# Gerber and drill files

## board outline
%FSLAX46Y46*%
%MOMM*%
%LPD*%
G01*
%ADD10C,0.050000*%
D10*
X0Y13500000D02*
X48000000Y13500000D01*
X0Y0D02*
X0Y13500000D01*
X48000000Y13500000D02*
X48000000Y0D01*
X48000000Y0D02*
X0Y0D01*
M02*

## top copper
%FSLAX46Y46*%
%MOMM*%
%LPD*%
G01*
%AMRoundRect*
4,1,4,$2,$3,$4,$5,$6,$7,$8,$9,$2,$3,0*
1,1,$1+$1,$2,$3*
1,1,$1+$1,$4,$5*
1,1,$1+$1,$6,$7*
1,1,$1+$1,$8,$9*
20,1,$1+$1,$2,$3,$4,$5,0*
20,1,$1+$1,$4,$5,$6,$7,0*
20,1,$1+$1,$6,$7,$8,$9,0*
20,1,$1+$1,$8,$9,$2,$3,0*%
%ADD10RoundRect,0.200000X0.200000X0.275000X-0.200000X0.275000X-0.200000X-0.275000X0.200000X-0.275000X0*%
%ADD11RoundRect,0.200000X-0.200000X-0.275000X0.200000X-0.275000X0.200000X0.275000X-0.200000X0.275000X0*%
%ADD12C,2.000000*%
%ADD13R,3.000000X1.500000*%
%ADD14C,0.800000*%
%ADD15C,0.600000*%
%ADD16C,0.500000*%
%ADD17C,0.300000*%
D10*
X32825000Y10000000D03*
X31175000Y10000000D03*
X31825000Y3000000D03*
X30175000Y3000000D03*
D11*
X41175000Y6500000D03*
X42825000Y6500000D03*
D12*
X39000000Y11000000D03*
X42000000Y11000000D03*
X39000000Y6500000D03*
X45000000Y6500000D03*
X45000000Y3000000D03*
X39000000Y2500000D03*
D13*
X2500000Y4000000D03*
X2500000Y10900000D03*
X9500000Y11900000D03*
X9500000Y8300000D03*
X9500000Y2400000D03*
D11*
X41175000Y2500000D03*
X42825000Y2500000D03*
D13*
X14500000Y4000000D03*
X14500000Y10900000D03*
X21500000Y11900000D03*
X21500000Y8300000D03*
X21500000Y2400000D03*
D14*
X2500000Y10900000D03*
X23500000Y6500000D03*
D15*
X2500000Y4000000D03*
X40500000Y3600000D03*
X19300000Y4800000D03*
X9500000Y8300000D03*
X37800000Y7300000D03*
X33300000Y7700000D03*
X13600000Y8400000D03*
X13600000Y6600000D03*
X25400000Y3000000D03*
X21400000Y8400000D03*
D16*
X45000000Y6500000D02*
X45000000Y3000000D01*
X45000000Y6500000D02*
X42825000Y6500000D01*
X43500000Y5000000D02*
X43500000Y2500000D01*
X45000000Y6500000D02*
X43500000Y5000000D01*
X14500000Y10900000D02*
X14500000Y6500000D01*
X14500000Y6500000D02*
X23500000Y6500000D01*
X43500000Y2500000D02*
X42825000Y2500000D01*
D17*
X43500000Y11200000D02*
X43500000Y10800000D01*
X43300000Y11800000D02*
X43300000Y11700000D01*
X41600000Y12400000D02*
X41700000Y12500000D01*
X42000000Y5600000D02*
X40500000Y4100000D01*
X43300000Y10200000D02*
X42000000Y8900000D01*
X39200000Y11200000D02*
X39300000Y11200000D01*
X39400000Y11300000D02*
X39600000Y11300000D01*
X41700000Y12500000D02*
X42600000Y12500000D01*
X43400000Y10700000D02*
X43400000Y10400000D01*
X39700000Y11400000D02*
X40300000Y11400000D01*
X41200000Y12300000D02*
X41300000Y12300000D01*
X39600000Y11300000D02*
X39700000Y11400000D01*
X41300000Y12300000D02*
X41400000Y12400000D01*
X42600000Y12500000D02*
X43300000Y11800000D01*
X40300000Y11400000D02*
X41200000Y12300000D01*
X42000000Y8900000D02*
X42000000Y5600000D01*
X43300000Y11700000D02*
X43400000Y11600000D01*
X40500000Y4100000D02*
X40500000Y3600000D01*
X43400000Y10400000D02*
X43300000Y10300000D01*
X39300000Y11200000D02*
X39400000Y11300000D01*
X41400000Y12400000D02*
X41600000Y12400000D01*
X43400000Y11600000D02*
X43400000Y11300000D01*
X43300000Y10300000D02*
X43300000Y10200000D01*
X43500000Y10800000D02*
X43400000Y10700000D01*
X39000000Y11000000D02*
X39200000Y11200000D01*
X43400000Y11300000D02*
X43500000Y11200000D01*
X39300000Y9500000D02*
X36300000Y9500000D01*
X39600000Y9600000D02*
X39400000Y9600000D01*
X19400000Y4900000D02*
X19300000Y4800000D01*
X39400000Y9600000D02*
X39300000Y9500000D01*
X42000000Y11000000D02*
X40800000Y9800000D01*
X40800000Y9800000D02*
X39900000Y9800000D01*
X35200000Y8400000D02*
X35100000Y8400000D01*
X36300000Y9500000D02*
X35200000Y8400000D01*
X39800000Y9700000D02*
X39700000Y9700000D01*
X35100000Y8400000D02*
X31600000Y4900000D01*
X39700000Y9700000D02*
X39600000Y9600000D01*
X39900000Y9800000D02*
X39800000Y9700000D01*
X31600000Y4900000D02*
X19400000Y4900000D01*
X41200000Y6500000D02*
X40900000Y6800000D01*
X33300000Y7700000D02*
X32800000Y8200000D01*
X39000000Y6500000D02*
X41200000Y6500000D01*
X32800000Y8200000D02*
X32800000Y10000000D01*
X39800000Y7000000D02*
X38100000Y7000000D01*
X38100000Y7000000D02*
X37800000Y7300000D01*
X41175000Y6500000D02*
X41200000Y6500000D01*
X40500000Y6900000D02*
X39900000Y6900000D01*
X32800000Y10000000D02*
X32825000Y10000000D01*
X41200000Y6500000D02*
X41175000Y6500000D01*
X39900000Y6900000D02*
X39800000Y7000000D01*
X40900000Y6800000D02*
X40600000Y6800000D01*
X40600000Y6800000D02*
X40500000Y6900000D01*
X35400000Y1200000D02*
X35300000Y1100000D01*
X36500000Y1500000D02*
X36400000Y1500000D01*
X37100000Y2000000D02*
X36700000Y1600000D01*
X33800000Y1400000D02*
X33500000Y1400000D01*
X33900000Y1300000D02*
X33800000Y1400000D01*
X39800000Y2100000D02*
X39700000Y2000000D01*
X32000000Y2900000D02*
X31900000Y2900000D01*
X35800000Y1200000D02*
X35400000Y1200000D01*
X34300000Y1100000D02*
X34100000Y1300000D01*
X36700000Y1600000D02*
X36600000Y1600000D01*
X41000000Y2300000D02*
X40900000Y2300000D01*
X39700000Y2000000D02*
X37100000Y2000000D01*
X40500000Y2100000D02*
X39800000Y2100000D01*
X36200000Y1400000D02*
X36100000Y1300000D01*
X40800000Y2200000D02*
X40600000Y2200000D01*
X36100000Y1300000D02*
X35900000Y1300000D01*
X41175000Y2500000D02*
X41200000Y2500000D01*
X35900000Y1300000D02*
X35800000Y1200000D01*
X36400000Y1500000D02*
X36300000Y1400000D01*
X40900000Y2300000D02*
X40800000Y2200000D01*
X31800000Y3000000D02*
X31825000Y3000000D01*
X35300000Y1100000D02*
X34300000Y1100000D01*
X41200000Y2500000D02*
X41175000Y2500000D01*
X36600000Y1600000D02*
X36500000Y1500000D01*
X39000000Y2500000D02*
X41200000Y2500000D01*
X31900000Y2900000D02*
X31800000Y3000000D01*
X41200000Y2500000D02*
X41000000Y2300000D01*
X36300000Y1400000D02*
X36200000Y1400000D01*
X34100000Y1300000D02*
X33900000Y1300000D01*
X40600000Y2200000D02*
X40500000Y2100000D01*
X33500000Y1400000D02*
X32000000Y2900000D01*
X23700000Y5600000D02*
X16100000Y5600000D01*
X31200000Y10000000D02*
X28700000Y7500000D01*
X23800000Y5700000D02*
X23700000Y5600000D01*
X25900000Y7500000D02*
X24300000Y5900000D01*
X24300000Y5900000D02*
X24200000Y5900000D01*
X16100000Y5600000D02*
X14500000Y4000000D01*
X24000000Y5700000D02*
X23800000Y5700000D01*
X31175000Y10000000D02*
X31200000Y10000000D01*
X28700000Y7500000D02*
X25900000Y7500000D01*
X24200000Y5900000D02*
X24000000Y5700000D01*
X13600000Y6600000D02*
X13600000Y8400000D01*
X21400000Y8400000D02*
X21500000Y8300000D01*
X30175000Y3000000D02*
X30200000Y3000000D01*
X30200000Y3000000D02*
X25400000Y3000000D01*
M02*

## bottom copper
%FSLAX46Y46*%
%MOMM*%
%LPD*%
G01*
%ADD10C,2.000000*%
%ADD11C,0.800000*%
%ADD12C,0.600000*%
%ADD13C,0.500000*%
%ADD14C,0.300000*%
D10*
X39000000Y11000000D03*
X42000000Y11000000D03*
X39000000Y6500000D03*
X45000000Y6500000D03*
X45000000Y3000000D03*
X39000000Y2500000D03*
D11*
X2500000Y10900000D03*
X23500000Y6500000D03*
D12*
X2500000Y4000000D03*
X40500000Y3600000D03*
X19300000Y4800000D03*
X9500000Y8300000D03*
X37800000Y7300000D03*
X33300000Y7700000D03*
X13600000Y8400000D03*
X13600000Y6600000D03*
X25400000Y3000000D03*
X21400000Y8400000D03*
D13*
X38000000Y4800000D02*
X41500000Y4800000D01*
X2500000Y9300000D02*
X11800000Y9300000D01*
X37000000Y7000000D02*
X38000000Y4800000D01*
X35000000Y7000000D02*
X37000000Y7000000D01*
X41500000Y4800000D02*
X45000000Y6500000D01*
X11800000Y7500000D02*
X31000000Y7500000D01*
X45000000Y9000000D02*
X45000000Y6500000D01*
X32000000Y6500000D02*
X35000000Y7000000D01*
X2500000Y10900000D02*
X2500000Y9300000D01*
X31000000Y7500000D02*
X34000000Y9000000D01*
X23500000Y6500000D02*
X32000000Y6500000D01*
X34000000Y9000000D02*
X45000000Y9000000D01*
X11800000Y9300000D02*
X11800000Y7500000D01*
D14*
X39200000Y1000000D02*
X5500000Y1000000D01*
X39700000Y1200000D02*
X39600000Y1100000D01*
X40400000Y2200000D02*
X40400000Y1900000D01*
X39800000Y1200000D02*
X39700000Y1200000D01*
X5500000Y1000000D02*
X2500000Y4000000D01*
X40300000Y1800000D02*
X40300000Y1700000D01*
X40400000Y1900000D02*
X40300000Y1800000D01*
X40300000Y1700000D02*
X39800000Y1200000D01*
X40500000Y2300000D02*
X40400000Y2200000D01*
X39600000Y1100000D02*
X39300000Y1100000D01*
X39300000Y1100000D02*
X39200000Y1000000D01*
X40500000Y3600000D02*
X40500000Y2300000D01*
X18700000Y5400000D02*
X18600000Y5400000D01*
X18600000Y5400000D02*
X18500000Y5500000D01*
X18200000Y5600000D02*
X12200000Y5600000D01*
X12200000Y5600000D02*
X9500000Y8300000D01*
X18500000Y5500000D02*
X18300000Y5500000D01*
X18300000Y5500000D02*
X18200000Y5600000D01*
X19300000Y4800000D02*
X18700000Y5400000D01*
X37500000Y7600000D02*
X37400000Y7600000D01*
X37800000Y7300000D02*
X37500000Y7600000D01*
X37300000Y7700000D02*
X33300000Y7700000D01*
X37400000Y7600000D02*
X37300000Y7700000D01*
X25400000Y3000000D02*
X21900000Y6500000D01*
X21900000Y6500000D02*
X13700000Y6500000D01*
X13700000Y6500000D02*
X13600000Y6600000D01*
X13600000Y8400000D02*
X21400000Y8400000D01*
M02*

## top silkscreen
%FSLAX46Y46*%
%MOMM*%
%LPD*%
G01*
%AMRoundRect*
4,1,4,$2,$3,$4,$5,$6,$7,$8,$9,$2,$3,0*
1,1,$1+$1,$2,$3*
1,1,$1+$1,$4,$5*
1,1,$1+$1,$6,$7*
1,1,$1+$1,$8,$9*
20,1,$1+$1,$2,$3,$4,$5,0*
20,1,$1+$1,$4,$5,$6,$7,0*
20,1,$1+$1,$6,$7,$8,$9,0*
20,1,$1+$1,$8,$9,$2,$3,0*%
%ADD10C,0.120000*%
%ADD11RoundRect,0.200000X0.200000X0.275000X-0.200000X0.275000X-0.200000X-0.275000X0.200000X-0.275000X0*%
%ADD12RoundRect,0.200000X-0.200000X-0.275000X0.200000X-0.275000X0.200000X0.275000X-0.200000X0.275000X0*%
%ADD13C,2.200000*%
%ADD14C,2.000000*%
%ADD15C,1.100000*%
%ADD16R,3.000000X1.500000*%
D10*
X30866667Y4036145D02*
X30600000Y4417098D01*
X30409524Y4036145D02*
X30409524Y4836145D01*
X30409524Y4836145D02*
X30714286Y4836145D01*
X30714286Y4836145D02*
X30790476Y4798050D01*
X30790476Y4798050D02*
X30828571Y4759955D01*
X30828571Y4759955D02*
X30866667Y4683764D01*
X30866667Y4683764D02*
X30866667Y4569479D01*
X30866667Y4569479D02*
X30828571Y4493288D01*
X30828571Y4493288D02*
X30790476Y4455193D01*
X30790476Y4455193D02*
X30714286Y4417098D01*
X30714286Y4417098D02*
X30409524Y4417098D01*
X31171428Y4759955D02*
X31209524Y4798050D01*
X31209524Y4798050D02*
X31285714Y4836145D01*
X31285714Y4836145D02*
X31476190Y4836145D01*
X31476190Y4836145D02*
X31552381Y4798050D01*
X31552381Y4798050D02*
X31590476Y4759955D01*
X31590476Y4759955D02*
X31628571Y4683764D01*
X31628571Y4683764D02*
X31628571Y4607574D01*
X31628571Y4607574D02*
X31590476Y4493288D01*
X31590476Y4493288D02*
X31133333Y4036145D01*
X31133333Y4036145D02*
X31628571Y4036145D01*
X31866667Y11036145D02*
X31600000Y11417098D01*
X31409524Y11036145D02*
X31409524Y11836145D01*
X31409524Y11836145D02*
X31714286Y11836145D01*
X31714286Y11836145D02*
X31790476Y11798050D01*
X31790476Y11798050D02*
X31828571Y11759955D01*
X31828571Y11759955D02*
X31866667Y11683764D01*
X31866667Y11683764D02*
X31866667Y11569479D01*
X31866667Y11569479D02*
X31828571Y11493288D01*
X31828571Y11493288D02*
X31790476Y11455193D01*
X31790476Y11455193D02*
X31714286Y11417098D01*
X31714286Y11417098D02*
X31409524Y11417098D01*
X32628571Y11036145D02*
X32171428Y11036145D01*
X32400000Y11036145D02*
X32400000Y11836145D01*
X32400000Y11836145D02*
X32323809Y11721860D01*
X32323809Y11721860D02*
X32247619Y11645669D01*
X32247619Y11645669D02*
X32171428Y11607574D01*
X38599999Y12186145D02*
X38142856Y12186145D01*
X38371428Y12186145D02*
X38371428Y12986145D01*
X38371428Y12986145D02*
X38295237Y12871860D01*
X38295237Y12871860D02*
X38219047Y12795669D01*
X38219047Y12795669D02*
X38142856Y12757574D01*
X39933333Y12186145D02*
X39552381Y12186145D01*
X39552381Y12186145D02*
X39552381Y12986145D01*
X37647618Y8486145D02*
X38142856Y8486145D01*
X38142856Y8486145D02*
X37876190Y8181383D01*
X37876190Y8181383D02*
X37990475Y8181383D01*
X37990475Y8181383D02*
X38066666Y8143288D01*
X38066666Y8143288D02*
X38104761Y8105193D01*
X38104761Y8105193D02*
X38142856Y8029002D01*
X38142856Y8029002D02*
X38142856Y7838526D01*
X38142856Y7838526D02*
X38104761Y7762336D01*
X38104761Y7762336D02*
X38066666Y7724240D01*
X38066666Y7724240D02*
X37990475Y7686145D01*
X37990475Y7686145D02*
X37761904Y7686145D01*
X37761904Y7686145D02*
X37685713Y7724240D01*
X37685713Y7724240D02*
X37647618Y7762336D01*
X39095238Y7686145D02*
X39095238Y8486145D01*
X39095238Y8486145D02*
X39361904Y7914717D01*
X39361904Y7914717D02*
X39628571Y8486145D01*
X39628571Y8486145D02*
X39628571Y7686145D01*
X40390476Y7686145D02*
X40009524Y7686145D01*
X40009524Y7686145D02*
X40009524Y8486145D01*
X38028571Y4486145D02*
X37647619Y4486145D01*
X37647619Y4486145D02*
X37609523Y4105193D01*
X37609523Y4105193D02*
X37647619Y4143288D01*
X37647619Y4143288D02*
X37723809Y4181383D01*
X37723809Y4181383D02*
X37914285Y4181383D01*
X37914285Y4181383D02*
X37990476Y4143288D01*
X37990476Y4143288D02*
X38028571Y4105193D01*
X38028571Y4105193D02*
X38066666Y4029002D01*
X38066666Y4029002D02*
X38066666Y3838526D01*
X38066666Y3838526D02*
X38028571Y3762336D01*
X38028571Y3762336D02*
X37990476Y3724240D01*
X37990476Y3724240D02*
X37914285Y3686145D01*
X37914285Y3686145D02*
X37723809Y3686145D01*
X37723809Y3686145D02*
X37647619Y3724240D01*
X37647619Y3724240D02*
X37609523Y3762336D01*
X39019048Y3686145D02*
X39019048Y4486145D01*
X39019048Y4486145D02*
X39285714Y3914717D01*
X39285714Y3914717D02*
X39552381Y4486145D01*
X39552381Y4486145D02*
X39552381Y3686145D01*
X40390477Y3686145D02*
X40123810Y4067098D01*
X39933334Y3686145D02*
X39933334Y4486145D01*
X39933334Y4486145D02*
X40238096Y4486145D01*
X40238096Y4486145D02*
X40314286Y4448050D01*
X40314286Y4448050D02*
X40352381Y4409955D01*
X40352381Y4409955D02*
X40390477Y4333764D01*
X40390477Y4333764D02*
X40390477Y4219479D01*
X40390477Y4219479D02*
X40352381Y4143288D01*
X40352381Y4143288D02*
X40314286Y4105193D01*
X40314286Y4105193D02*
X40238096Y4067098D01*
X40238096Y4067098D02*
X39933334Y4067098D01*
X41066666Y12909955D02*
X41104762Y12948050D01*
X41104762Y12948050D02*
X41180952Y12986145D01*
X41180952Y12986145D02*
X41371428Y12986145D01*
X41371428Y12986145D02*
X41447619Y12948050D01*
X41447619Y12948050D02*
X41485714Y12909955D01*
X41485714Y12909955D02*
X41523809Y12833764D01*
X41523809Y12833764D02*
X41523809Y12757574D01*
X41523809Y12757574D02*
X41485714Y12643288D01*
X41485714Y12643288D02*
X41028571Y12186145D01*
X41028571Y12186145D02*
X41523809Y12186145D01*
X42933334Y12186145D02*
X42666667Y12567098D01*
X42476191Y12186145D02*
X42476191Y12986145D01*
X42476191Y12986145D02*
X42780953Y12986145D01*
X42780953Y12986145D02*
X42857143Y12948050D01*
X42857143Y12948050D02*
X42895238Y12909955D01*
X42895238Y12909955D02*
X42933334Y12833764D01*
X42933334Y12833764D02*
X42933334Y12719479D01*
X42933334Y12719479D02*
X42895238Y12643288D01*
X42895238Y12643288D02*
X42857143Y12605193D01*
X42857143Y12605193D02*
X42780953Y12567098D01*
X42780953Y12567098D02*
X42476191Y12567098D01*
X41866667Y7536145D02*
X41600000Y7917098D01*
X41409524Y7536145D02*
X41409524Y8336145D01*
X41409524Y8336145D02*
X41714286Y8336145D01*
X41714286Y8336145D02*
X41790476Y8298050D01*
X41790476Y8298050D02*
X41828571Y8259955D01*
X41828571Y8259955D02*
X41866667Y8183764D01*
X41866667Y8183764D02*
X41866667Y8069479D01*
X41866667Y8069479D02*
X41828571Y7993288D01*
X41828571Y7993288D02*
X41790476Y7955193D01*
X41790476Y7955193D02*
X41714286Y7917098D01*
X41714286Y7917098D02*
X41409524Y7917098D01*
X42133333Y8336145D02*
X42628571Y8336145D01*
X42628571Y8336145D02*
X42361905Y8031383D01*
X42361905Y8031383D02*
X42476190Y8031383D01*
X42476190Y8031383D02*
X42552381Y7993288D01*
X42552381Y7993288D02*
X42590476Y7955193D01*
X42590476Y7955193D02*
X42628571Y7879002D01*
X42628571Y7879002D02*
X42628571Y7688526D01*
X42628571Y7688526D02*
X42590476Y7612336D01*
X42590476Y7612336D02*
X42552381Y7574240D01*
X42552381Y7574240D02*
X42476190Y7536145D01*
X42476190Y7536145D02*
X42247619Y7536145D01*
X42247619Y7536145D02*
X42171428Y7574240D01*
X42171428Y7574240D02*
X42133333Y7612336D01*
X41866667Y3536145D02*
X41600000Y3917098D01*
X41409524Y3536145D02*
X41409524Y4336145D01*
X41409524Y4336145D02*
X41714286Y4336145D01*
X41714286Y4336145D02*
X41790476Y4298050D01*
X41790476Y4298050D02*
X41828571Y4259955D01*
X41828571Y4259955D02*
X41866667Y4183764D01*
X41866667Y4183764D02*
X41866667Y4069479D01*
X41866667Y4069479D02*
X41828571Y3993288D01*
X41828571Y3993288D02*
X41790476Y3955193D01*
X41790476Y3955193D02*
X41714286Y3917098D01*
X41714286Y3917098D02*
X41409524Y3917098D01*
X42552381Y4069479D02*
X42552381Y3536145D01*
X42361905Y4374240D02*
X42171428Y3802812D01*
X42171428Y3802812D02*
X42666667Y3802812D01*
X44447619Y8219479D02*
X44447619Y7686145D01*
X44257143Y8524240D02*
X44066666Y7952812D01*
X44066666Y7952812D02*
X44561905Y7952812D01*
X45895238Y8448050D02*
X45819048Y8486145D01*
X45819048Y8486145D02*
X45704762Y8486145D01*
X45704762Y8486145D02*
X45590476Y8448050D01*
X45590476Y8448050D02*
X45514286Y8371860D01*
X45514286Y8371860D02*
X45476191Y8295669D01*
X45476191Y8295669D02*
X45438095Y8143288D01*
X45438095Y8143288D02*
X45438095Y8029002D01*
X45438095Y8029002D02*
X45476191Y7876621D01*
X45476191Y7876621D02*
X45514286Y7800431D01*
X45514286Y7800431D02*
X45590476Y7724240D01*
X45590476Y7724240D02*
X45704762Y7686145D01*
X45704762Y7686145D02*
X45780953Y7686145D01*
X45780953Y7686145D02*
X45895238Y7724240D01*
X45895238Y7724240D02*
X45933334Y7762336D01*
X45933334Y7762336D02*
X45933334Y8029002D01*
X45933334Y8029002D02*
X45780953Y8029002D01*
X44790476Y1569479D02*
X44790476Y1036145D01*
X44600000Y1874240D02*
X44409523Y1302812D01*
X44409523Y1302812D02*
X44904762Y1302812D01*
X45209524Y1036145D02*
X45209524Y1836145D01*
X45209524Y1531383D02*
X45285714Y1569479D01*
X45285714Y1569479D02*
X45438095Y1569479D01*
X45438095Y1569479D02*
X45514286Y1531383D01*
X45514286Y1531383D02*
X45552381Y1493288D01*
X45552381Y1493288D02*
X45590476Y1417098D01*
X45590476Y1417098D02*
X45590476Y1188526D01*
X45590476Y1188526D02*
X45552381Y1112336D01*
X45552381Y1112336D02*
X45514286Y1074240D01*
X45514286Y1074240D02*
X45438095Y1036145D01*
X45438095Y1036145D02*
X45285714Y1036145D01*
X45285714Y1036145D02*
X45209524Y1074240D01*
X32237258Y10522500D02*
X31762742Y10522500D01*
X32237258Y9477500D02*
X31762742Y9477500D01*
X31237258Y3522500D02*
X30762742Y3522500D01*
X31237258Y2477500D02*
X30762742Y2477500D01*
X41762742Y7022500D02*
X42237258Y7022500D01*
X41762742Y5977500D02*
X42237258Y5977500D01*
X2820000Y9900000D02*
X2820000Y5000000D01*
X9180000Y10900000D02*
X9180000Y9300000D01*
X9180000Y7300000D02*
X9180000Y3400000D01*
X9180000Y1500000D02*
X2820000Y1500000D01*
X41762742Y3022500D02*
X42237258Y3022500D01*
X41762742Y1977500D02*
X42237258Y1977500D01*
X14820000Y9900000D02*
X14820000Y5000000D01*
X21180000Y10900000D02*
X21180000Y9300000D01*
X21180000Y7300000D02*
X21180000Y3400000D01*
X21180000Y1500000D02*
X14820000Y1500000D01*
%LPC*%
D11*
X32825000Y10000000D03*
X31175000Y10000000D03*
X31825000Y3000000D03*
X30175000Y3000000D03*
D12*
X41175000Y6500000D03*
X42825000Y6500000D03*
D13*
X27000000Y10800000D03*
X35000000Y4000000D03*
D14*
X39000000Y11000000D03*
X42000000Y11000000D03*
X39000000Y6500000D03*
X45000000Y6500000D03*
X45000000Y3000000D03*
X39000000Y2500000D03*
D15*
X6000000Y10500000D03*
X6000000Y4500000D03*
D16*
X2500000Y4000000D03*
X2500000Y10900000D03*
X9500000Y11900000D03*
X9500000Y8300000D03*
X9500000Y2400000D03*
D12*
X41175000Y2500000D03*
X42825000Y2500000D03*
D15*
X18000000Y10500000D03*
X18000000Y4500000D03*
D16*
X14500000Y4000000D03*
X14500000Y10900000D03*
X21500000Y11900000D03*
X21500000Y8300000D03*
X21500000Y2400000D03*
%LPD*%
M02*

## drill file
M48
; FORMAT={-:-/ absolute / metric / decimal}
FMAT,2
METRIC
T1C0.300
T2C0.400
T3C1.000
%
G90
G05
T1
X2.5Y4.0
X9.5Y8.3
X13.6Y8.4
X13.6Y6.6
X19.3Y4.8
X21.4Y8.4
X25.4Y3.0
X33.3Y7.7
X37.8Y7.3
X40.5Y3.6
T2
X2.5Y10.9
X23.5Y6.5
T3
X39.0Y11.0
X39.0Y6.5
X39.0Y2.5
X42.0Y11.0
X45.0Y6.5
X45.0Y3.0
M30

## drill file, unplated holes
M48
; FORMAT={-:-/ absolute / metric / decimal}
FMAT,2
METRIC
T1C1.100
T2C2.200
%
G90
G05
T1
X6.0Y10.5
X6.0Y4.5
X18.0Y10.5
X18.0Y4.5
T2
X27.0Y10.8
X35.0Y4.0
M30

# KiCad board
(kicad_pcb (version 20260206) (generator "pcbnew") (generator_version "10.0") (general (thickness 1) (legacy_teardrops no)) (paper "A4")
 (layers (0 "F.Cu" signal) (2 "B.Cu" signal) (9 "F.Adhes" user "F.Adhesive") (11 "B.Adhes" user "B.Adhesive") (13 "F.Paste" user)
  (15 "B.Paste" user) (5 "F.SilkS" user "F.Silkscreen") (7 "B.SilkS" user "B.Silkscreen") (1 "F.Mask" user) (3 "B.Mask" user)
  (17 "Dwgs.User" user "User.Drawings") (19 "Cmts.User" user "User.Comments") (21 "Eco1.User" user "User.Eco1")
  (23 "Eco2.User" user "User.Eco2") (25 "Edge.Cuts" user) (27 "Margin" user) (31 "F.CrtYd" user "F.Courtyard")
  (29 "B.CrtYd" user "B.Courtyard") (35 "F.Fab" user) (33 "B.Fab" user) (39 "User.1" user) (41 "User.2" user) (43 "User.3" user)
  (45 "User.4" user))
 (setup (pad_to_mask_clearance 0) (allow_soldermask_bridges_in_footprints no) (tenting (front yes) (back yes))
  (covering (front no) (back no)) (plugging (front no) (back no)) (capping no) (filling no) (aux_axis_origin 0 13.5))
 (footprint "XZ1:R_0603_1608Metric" (layer "F.Cu") (at 32 3.5 180)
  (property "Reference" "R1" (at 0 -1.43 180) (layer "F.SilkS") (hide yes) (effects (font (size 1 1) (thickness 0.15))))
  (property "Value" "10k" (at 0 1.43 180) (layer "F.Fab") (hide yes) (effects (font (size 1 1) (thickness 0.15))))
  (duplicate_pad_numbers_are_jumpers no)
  (fp_line (start -0.237258 0.5225) (end 0.237258 0.5225) (stroke (width 0.12) (type solid)) (layer "F.SilkS"))
  (fp_line (start -0.237258 -0.5225) (end 0.237258 -0.5225) (stroke (width 0.12) (type solid)) (layer "F.SilkS"))
  (pad "1" smd roundrect (at -0.825 0 180) (size 0.8 0.95) (layers "F.Cu" "F.Mask" "F.Paste") (roundrect_rratio 0.25) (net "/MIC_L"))
  (pad "2" smd roundrect (at 0.825 0 180) (size 0.8 0.95) (layers "F.Cu" "F.Mask" "F.Paste") (roundrect_rratio 0.25) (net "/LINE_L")))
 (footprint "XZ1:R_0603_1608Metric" (layer "F.Cu") (at 31 10.5 180)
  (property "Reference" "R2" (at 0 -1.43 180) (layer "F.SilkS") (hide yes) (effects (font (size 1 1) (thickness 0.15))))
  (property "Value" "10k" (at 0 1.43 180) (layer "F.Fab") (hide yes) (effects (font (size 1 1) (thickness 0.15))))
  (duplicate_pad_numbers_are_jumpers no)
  (fp_line (start -0.237258 0.5225) (end 0.237258 0.5225) (stroke (width 0.12) (type solid)) (layer "F.SilkS"))
  (fp_line (start -0.237258 -0.5225) (end 0.237258 -0.5225) (stroke (width 0.12) (type solid)) (layer "F.SilkS"))
  (pad "1" smd roundrect (at -0.825 0 180) (size 0.8 0.95) (layers "F.Cu" "F.Mask" "F.Paste") (roundrect_rratio 0.25) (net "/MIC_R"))
  (pad "2" smd roundrect (at 0.825 0 180) (size 0.8 0.95) (layers "F.Cu" "F.Mask" "F.Paste") (roundrect_rratio 0.25) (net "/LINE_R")))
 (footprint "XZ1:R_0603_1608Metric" (layer "F.Cu") (at 42 7)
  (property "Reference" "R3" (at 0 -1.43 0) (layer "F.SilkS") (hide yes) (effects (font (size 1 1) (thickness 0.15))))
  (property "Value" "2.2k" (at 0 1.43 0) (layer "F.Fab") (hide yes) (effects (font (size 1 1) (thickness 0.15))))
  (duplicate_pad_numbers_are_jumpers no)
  (fp_line (start -0.237258 -0.5225) (end 0.237258 -0.5225) (stroke (width 0.12) (type solid)) (layer "F.SilkS"))
  (fp_line (start -0.237258 0.5225) (end 0.237258 0.5225) (stroke (width 0.12) (type solid)) (layer "F.SilkS"))
  (pad "1" smd roundrect (at -0.825 0) (size 0.8 0.95) (layers "F.Cu" "F.Mask" "F.Paste") (roundrect_rratio 0.25) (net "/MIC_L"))
  (pad "2" smd roundrect (at 0.825 0) (size 0.8 0.95) (layers "F.Cu" "F.Mask" "F.Paste") (roundrect_rratio 0.25) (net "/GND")))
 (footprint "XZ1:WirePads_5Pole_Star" (layer "F.Cu") (at 0 0)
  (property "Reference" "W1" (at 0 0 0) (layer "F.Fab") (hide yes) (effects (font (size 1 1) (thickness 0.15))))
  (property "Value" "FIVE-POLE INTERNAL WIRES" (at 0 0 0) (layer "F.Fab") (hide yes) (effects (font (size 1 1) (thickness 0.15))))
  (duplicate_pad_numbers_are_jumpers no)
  (pad "" np_thru_hole circle (at 27 2.7) (size 2.2 2.2) (drill 2.2) (layers "*.Cu" "*.Mask"))
  (pad "" np_thru_hole circle (at 35 9.5) (size 2.2 2.2) (drill 2.2) (layers "*.Cu" "*.Mask"))
  (pad "1" thru_hole circle (at 39 2.5) (size 2 2) (drill 1) (layers "*.Cu" "*.Mask") (remove_unused_layers no) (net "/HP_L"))
  (pad "2" thru_hole circle (at 42 2.5) (size 2 2) (drill 1) (layers "*.Cu" "*.Mask") (remove_unused_layers no) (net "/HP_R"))
  (pad "3" thru_hole circle (at 39 7) (size 2 2) (drill 1) (layers "*.Cu" "*.Mask") (remove_unused_layers no) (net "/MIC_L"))
  (pad "4" thru_hole circle (at 45 7) (size 2 2) (drill 1) (layers "*.Cu" "*.Mask") (remove_unused_layers no) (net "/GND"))
  (pad "4b" thru_hole circle (at 45 10.5) (size 2 2) (drill 1) (layers "*.Cu" "*.Mask") (remove_unused_layers no) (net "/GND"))
  (pad "5" thru_hole circle (at 39 11) (size 2 2) (drill 1) (layers "*.Cu" "*.Mask") (remove_unused_layers no) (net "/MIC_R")))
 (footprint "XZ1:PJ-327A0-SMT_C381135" (layer "F.Cu") (at 6 6 -90)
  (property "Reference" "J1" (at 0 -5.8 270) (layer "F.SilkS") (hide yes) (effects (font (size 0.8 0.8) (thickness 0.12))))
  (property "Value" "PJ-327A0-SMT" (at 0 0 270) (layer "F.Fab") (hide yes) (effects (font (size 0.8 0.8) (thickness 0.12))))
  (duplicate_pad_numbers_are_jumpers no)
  (fp_line (start -2.4 3.18) (end 2.5 3.18) (stroke (width 0.12) (type solid)) (layer "F.SilkS"))
  (fp_line (start -3.4 -3.18) (end -1.8 -3.18) (stroke (width 0.12) (type solid)) (layer "F.SilkS"))
  (fp_line (start 0.2 -3.18) (end 4.1 -3.18) (stroke (width 0.12) (type solid)) (layer "F.SilkS"))
  (fp_line (start 6 -3.18) (end 6 3.18) (stroke (width 0.12) (type solid)) (layer "F.SilkS"))
  (pad "" np_thru_hole circle (at -3 0 270) (size 1.1 1.1) (drill 1.1) (layers "*.Cu" "*.Mask"))
  (pad "" np_thru_hole circle (at 3 0 270) (size 1.1 1.1) (drill 1.1) (layers "*.Cu" "*.Mask"))
  (pad "2" smd rect (at 3.5 3.5 270) (size 1.5 3) (layers "F.Cu" "F.Mask" "F.Paste") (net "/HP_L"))
  (pad "3" smd rect (at -3.4 3.5 270) (size 1.5 3) (layers "F.Cu" "F.Mask" "F.Paste") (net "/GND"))
  (pad "4" smd rect (at -4.4 -3.5 270) (size 1.5 3) (layers "F.Cu" "F.Mask" "F.Paste") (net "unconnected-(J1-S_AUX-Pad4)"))
  (pad "5" smd rect (at -0.8 -3.5 270) (size 1.5 3) (layers "F.Cu" "F.Mask" "F.Paste") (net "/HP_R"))
  (pad "6" smd rect (at 5.1 -3.5 270) (size 1.5 3) (layers "F.Cu" "F.Mask" "F.Paste") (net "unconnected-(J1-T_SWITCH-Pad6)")))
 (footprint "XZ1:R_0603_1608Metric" (layer "F.Cu") (at 42 11)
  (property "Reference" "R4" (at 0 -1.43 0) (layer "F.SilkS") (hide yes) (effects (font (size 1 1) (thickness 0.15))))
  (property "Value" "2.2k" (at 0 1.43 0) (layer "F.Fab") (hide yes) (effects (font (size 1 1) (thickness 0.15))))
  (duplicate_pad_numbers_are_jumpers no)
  (fp_line (start -0.237258 -0.5225) (end 0.237258 -0.5225) (stroke (width 0.12) (type solid)) (layer "F.SilkS"))
  (fp_line (start -0.237258 0.5225) (end 0.237258 0.5225) (stroke (width 0.12) (type solid)) (layer "F.SilkS"))
  (pad "1" smd roundrect (at -0.825 0) (size 0.8 0.95) (layers "F.Cu" "F.Mask" "F.Paste") (roundrect_rratio 0.25) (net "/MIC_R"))
  (pad "2" smd roundrect (at 0.825 0) (size 0.8 0.95) (layers "F.Cu" "F.Mask" "F.Paste") (roundrect_rratio 0.25) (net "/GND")))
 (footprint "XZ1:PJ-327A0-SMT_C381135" (layer "F.Cu") (at 18 6 -90)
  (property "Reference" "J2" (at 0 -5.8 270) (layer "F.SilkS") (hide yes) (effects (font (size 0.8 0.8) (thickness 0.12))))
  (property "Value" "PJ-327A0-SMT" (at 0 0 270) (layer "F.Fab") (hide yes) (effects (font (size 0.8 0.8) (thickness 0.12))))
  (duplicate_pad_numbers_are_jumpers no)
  (fp_line (start -2.4 3.18) (end 2.5 3.18) (stroke (width 0.12) (type solid)) (layer "F.SilkS"))
  (fp_line (start -3.4 -3.18) (end -1.8 -3.18) (stroke (width 0.12) (type solid)) (layer "F.SilkS"))
  (fp_line (start 0.2 -3.18) (end 4.1 -3.18) (stroke (width 0.12) (type solid)) (layer "F.SilkS"))
  (fp_line (start 6 -3.18) (end 6 3.18) (stroke (width 0.12) (type solid)) (layer "F.SilkS"))
  (pad "" np_thru_hole circle (at -3 0 270) (size 1.1 1.1) (drill 1.1) (layers "*.Cu" "*.Mask"))
  (pad "" np_thru_hole circle (at 3 0 270) (size 1.1 1.1) (drill 1.1) (layers "*.Cu" "*.Mask"))
  (pad "2" smd rect (at 3.5 3.5 270) (size 1.5 3) (layers "F.Cu" "F.Mask" "F.Paste") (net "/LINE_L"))
  (pad "3" smd rect (at -3.4 3.5 270) (size 1.5 3) (layers "F.Cu" "F.Mask" "F.Paste") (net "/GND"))
  (pad "4" smd rect (at -4.4 -3.5 270) (size 1.5 3) (layers "F.Cu" "F.Mask" "F.Paste") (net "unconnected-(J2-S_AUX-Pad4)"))
  (pad "5" smd rect (at -0.8 -3.5 270) (size 1.5 3) (layers "F.Cu" "F.Mask" "F.Paste") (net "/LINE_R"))
  (pad "6" smd rect (at 5.1 -3.5 270) (size 1.5 3) (layers "F.Cu" "F.Mask" "F.Paste") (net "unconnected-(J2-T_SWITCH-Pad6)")))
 (gr_line (start 0 0) (end 48 0) (stroke (width 0.05) (type default)) (layer "Edge.Cuts"))
 (gr_line (start 0 13.5) (end 0 0) (stroke (width 0.05) (type default)) (layer "Edge.Cuts"))
 (gr_line (start 48 0) (end 48 13.5) (stroke (width 0.05) (type default)) (layer "Edge.Cuts"))
 (gr_line (start 48 13.5) (end 0 13.5) (stroke (width 0.05) (type default)) (layer "Edge.Cuts"))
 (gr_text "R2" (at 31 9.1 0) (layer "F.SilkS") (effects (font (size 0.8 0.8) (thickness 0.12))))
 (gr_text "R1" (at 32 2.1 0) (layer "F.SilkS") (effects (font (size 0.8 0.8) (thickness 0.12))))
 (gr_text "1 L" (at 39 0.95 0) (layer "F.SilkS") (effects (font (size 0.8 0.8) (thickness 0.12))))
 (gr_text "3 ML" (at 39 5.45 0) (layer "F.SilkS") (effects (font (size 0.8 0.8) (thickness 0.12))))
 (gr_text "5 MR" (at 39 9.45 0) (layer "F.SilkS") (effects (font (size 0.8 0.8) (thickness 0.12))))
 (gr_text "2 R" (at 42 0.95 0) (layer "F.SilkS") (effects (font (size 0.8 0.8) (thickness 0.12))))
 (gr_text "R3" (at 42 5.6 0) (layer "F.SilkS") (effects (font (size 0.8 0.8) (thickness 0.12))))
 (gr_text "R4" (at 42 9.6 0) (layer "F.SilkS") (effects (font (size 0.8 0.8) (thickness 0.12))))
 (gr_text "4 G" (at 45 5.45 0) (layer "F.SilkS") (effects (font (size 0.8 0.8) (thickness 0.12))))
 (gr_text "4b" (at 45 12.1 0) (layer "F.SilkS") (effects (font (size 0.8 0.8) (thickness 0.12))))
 (segment (start 45 7) (end 45 10.5) (width 0.5) (layer "F.Cu") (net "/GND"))
 (segment (start 45 7) (end 42.825 7) (width 0.5) (layer "F.Cu") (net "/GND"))
 (segment (start 43.5 8.5) (end 43.5 11) (width 0.5) (layer "F.Cu") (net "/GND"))
 (segment (start 45 7) (end 43.5 8.5) (width 0.5) (layer "F.Cu") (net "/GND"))
 (segment (start 14.5 2.6) (end 14.5 7) (width 0.5) (layer "F.Cu") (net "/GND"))
 (segment (start 14.5 7) (end 23.5 7) (width 0.5) (layer "F.Cu") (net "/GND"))
 (segment (start 43.5 11) (end 42.825 11) (width 0.5) (layer "F.Cu") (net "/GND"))
 (via (at 2.5 2.6) (size 0.8) (drill 0.4) (layers "F.Cu" "B.Cu") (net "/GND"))
 (via (at 23.5 7) (size 0.8) (drill 0.4) (layers "F.Cu" "B.Cu") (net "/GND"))
 (segment (start 38 8.7) (end 41.5 8.7) (width 0.5) (layer "B.Cu") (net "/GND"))
 (segment (start 2.5 4.2) (end 11.8 4.2) (width 0.5) (layer "B.Cu") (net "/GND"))
 (segment (start 37 6.5) (end 38 8.7) (width 0.5) (layer "B.Cu") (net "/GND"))
 (segment (start 35 6.5) (end 37 6.5) (width 0.5) (layer "B.Cu") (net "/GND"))
 (segment (start 41.5 8.7) (end 45 7) (width 0.5) (layer "B.Cu") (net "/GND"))
 (segment (start 11.8 6) (end 31 6) (width 0.5) (layer "B.Cu") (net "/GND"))
 (segment (start 45 4.5) (end 45 7) (width 0.5) (layer "B.Cu") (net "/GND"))
 (segment (start 32 7) (end 35 6.5) (width 0.5) (layer "B.Cu") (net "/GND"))
 (segment (start 2.5 2.6) (end 2.5 4.2) (width 0.5) (layer "B.Cu") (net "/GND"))
 (segment (start 31 6) (end 34 4.5) (width 0.5) (layer "B.Cu") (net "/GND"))
 (segment (start 23.5 7) (end 32 7) (width 0.5) (layer "B.Cu") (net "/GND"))
 (segment (start 34 4.5) (end 45 4.5) (width 0.5) (layer "B.Cu") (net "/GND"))
 (segment (start 11.8 4.2) (end 11.8 6) (width 0.5) (layer "B.Cu") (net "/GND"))
 (segment (start 43.5 2.3) (end 43.5 2.7) (width 0.3) (layer "F.Cu") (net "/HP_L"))
 (segment (start 43.3 1.7) (end 43.3 1.8) (width 0.3) (layer "F.Cu") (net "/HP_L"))
 (segment (start 41.6 1.1) (end 41.7 1) (width 0.3) (layer "F.Cu") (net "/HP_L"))
 (segment (start 42 7.9) (end 40.5 9.4) (width 0.3) (layer "F.Cu") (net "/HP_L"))
 (segment (start 43.3 3.3) (end 42 4.6) (width 0.3) (layer "F.Cu") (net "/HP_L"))
 (segment (start 39.2 2.3) (end 39.3 2.3) (width 0.3) (layer "F.Cu") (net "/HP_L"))
 (segment (start 39.4 2.2) (end 39.6 2.2) (width 0.3) (layer "F.Cu") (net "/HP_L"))
 (segment (start 41.7 1) (end 42.6 1) (width 0.3) (layer "F.Cu") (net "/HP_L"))
 (segment (start 43.4 2.8) (end 43.4 3.1) (width 0.3) (layer "F.Cu") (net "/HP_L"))
 (segment (start 39.7 2.1) (end 40.3 2.1) (width 0.3) (layer "F.Cu") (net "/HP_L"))
 (segment (start 41.2 1.2) (end 41.3 1.2) (width 0.3) (layer "F.Cu") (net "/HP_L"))
 (segment (start 39.6 2.2) (end 39.7 2.1) (width 0.3) (layer "F.Cu") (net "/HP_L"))
 (segment (start 41.3 1.2) (end 41.4 1.1) (width 0.3) (layer "F.Cu") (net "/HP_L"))
 (segment (start 42.6 1) (end 43.3 1.7) (width 0.3) (layer "F.Cu") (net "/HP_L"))
 (segment (start 40.3 2.1) (end 41.2 1.2) (width 0.3) (layer "F.Cu") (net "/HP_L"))
 (segment (start 42 4.6) (end 42 7.9) (width 0.3) (layer "F.Cu") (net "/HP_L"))
 (segment (start 43.3 1.8) (end 43.4 1.9) (width 0.3) (layer "F.Cu") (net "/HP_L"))
 (segment (start 40.5 9.4) (end 40.5 9.9) (width 0.3) (layer "F.Cu") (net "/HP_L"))
 (segment (start 43.4 3.1) (end 43.3 3.2) (width 0.3) (layer "F.Cu") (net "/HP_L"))
 (segment (start 39.3 2.3) (end 39.4 2.2) (width 0.3) (layer "F.Cu") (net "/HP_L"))
 (segment (start 41.4 1.1) (end 41.6 1.1) (width 0.3) (layer "F.Cu") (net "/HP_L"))
 (segment (start 43.4 1.9) (end 43.4 2.2) (width 0.3) (layer "F.Cu") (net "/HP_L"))
 (segment (start 43.3 3.2) (end 43.3 3.3) (width 0.3) (layer "F.Cu") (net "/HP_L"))
 (segment (start 43.5 2.7) (end 43.4 2.8) (width 0.3) (layer "F.Cu") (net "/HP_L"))
 (segment (start 39 2.5) (end 39.2 2.3) (width 0.3) (layer "F.Cu") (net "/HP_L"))
 (segment (start 43.4 2.2) (end 43.5 2.3) (width 0.3) (layer "F.Cu") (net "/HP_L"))
 (via (at 2.5 9.5) (size 0.6) (drill 0.3) (layers "F.Cu" "B.Cu") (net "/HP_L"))
 (via (at 40.5 9.9) (size 0.6) (drill 0.3) (layers "F.Cu" "B.Cu") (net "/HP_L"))
 (segment (start 39.2 12.5) (end 5.5 12.5) (width 0.3) (layer "B.Cu") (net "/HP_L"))
 (segment (start 39.7 12.3) (end 39.6 12.4) (width 0.3) (layer "B.Cu") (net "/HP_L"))
 (segment (start 40.4 11.3) (end 40.4 11.6) (width 0.3) (layer "B.Cu") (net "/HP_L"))
 (segment (start 39.8 12.3) (end 39.7 12.3) (width 0.3) (layer "B.Cu") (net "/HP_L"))
 (segment (start 5.5 12.5) (end 2.5 9.5) (width 0.3) (layer "B.Cu") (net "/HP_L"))
 (segment (start 40.3 11.7) (end 40.3 11.8) (width 0.3) (layer "B.Cu") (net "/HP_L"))
 (segment (start 40.4 11.6) (end 40.3 11.7) (width 0.3) (layer "B.Cu") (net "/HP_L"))
 (segment (start 40.3 11.8) (end 39.8 12.3) (width 0.3) (layer "B.Cu") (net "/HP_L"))
 (segment (start 40.5 11.2) (end 40.4 11.3) (width 0.3) (layer "B.Cu") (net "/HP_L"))
 (segment (start 39.6 12.4) (end 39.3 12.4) (width 0.3) (layer "B.Cu") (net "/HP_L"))
 (segment (start 39.3 12.4) (end 39.2 12.5) (width 0.3) (layer "B.Cu") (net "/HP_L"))
 (segment (start 40.5 9.9) (end 40.5 11.2) (width 0.3) (layer "B.Cu") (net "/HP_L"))
 (segment (start 39.3 4) (end 36.3 4) (width 0.3) (layer "F.Cu") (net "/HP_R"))
 (segment (start 39.6 3.9) (end 39.4 3.9) (width 0.3) (layer "F.Cu") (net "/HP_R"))
 (segment (start 19.4 8.6) (end 19.3 8.7) (width 0.3) (layer "F.Cu") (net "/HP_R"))
 (segment (start 39.4 3.9) (end 39.3 4) (width 0.3) (layer "F.Cu") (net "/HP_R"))
 (segment (start 42 2.5) (end 40.8 3.7) (width 0.3) (layer "F.Cu") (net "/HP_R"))
 (segment (start 40.8 3.7) (end 39.9 3.7) (width 0.3) (layer "F.Cu") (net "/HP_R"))
 (segment (start 35.2 5.1) (end 35.1 5.1) (width 0.3) (layer "F.Cu") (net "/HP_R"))
 (segment (start 36.3 4) (end 35.2 5.1) (width 0.3) (layer "F.Cu") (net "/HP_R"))
 (segment (start 39.8 3.8) (end 39.7 3.8) (width 0.3) (layer "F.Cu") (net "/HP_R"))
 (segment (start 35.1 5.1) (end 31.6 8.6) (width 0.3) (layer "F.Cu") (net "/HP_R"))
 (segment (start 39.7 3.8) (end 39.6 3.9) (width 0.3) (layer "F.Cu") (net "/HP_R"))
 (segment (start 39.9 3.7) (end 39.8 3.8) (width 0.3) (layer "F.Cu") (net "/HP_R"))
 (segment (start 31.6 8.6) (end 19.4 8.6) (width 0.3) (layer "F.Cu") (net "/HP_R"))
 (via (at 19.3 8.7) (size 0.6) (drill 0.3) (layers "F.Cu" "B.Cu") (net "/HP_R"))
 (via (at 9.5 5.2) (size 0.6) (drill 0.3) (layers "F.Cu" "B.Cu") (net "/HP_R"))
 (segment (start 18.7 8.1) (end 18.6 8.1) (width 0.3) (layer "B.Cu") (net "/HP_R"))
 (segment (start 18.6 8.1) (end 18.5 8) (width 0.3) (layer "B.Cu") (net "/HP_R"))
 (segment (start 18.2 7.9) (end 12.2 7.9) (width 0.3) (layer "B.Cu") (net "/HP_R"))
 (segment (start 12.2 7.9) (end 9.5 5.2) (width 0.3) (layer "B.Cu") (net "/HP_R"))
 (segment (start 18.5 8) (end 18.3 8) (width 0.3) (layer "B.Cu") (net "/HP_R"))
 (segment (start 18.3 8) (end 18.2 7.9) (width 0.3) (layer "B.Cu") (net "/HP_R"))
 (segment (start 19.3 8.7) (end 18.7 8.1) (width 0.3) (layer "B.Cu") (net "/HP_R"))
 (segment (start 41.2 7) (end 40.9 6.7) (width 0.3) (layer "F.Cu") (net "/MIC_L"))
 (segment (start 33.3 5.8) (end 32.8 5.3) (width 0.3) (layer "F.Cu") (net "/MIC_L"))
 (segment (start 39 7) (end 41.2 7) (width 0.3) (layer "F.Cu") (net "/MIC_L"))
 (segment (start 32.8 5.3) (end 32.8 3.5) (width 0.3) (layer "F.Cu") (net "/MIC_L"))
 (segment (start 39.8 6.5) (end 38.1 6.5) (width 0.3) (layer "F.Cu") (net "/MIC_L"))
 (segment (start 38.1 6.5) (end 37.8 6.2) (width 0.3) (layer "F.Cu") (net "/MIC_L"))
 (segment (start 41.175 7) (end 41.2 7) (width 0.3) (layer "F.Cu") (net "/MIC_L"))
 (segment (start 40.5 6.6) (end 39.9 6.6) (width 0.3) (layer "F.Cu") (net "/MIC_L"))
 (segment (start 32.8 3.5) (end 32.825 3.5) (width 0.3) (layer "F.Cu") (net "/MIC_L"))
 (segment (start 41.2 7) (end 41.175 7) (width 0.3) (layer "F.Cu") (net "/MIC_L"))
 (segment (start 39.9 6.6) (end 39.8 6.5) (width 0.3) (layer "F.Cu") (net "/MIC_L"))
 (segment (start 40.9 6.7) (end 40.6 6.7) (width 0.3) (layer "F.Cu") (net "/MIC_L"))
 (segment (start 40.6 6.7) (end 40.5 6.6) (width 0.3) (layer "F.Cu") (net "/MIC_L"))
 (via (at 37.8 6.2) (size 0.6) (drill 0.3) (layers "F.Cu" "B.Cu") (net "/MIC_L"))
 (via (at 33.3 5.8) (size 0.6) (drill 0.3) (layers "F.Cu" "B.Cu") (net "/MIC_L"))
 (segment (start 37.5 5.9) (end 37.4 5.9) (width 0.3) (layer "B.Cu") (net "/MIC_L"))
 (segment (start 37.8 6.2) (end 37.5 5.9) (width 0.3) (layer "B.Cu") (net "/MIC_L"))
 (segment (start 37.3 5.8) (end 33.3 5.8) (width 0.3) (layer "B.Cu") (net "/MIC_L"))
 (segment (start 37.4 5.9) (end 37.3 5.8) (width 0.3) (layer "B.Cu") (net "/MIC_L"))
 (segment (start 35.4 12.3) (end 35.3 12.4) (width 0.3) (layer "F.Cu") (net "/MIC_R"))
 (segment (start 36.5 12) (end 36.4 12) (width 0.3) (layer "F.Cu") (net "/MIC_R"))
 (segment (start 37.1 11.5) (end 36.7 11.9) (width 0.3) (layer "F.Cu") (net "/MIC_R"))
 (segment (start 33.8 12.1) (end 33.5 12.1) (width 0.3) (layer "F.Cu") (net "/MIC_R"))
 (segment (start 33.9 12.2) (end 33.8 12.1) (width 0.3) (layer "F.Cu") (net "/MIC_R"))
 (segment (start 39.8 11.4) (end 39.7 11.5) (width 0.3) (layer "F.Cu") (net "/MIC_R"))
 (segment (start 32 10.6) (end 31.9 10.6) (width 0.3) (layer "F.Cu") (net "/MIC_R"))
 (segment (start 35.8 12.3) (end 35.4 12.3) (width 0.3) (layer "F.Cu") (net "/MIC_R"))
 (segment (start 34.3 12.4) (end 34.1 12.2) (width 0.3) (layer "F.Cu") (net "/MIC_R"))
 (segment (start 36.7 11.9) (end 36.6 11.9) (width 0.3) (layer "F.Cu") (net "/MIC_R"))
 (segment (start 41 11.2) (end 40.9 11.2) (width 0.3) (layer "F.Cu") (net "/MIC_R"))
 (segment (start 39.7 11.5) (end 37.1 11.5) (width 0.3) (layer "F.Cu") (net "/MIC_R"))
 (segment (start 40.5 11.4) (end 39.8 11.4) (width 0.3) (layer "F.Cu") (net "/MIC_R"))
 (segment (start 36.2 12.1) (end 36.1 12.2) (width 0.3) (layer "F.Cu") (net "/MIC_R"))
 (segment (start 40.8 11.3) (end 40.6 11.3) (width 0.3) (layer "F.Cu") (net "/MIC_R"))
 (segment (start 36.1 12.2) (end 35.9 12.2) (width 0.3) (layer "F.Cu") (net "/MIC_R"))
 (segment (start 41.175 11) (end 41.2 11) (width 0.3) (layer "F.Cu") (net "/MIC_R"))
 (segment (start 35.9 12.2) (end 35.8 12.3) (width 0.3) (layer "F.Cu") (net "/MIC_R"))
 (segment (start 36.4 12) (end 36.3 12.1) (width 0.3) (layer "F.Cu") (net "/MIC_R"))
 (segment (start 40.9 11.2) (end 40.8 11.3) (width 0.3) (layer "F.Cu") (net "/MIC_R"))
 (segment (start 31.8 10.5) (end 31.825 10.5) (width 0.3) (layer "F.Cu") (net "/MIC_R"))
 (segment (start 35.3 12.4) (end 34.3 12.4) (width 0.3) (layer "F.Cu") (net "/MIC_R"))
 (segment (start 41.2 11) (end 41.175 11) (width 0.3) (layer "F.Cu") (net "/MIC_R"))
 (segment (start 36.6 11.9) (end 36.5 12) (width 0.3) (layer "F.Cu") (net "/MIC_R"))
 (segment (start 39 11) (end 41.2 11) (width 0.3) (layer "F.Cu") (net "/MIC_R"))
 (segment (start 31.9 10.6) (end 31.8 10.5) (width 0.3) (layer "F.Cu") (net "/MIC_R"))
 (segment (start 41.2 11) (end 41 11.2) (width 0.3) (layer "F.Cu") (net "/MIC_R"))
 (segment (start 36.3 12.1) (end 36.2 12.1) (width 0.3) (layer "F.Cu") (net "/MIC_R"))
 (segment (start 34.1 12.2) (end 33.9 12.2) (width 0.3) (layer "F.Cu") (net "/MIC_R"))
 (segment (start 40.6 11.3) (end 40.5 11.4) (width 0.3) (layer "F.Cu") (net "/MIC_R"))
 (segment (start 33.5 12.1) (end 32 10.6) (width 0.3) (layer "F.Cu") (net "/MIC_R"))
 (segment (start 23.7 7.9) (end 16.1 7.9) (width 0.3) (layer "F.Cu") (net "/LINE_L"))
 (segment (start 31.2 3.5) (end 28.7 6) (width 0.3) (layer "F.Cu") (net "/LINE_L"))
 (segment (start 23.8 7.8) (end 23.7 7.9) (width 0.3) (layer "F.Cu") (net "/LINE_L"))
 (segment (start 25.9 6) (end 24.3 7.6) (width 0.3) (layer "F.Cu") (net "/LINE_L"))
 (segment (start 24.3 7.6) (end 24.2 7.6) (width 0.3) (layer "F.Cu") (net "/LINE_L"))
 (segment (start 16.1 7.9) (end 14.5 9.5) (width 0.3) (layer "F.Cu") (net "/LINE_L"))
 (segment (start 24 7.8) (end 23.8 7.8) (width 0.3) (layer "F.Cu") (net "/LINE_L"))
 (segment (start 31.175 3.5) (end 31.2 3.5) (width 0.3) (layer "F.Cu") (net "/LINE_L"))
 (segment (start 28.7 6) (end 25.9 6) (width 0.3) (layer "F.Cu") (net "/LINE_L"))
 (segment (start 24.2 7.6) (end 24 7.8) (width 0.3) (layer "F.Cu") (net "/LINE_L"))
 (segment (start 13.6 6.9) (end 13.6 5.1) (width 0.3) (layer "F.Cu") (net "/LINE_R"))
 (segment (start 21.4 5.1) (end 21.5 5.2) (width 0.3) (layer "F.Cu") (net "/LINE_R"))
 (segment (start 30.175 10.5) (end 30.2 10.5) (width 0.3) (layer "F.Cu") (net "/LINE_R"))
 (segment (start 30.2 10.5) (end 25.4 10.5) (width 0.3) (layer "F.Cu") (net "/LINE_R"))
 (via (at 13.6 5.1) (size 0.6) (drill 0.3) (layers "F.Cu" "B.Cu") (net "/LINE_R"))
 (via (at 13.6 6.9) (size 0.6) (drill 0.3) (layers "F.Cu" "B.Cu") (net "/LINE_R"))
 (via (at 25.4 10.5) (size 0.6) (drill 0.3) (layers "F.Cu" "B.Cu") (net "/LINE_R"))
 (via (at 21.4 5.1) (size 0.6) (drill 0.3) (layers "F.Cu" "B.Cu") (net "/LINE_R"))
 (segment (start 25.4 10.5) (end 21.9 7) (width 0.3) (layer "B.Cu") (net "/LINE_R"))
 (segment (start 21.9 7) (end 13.7 7) (width 0.3) (layer "B.Cu") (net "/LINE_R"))
 (segment (start 13.7 7) (end 13.6 6.9) (width 0.3) (layer "B.Cu") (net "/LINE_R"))
 (segment (start 13.6 5.1) (end 21.4 5.1) (width 0.3) (layer "B.Cu") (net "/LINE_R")))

